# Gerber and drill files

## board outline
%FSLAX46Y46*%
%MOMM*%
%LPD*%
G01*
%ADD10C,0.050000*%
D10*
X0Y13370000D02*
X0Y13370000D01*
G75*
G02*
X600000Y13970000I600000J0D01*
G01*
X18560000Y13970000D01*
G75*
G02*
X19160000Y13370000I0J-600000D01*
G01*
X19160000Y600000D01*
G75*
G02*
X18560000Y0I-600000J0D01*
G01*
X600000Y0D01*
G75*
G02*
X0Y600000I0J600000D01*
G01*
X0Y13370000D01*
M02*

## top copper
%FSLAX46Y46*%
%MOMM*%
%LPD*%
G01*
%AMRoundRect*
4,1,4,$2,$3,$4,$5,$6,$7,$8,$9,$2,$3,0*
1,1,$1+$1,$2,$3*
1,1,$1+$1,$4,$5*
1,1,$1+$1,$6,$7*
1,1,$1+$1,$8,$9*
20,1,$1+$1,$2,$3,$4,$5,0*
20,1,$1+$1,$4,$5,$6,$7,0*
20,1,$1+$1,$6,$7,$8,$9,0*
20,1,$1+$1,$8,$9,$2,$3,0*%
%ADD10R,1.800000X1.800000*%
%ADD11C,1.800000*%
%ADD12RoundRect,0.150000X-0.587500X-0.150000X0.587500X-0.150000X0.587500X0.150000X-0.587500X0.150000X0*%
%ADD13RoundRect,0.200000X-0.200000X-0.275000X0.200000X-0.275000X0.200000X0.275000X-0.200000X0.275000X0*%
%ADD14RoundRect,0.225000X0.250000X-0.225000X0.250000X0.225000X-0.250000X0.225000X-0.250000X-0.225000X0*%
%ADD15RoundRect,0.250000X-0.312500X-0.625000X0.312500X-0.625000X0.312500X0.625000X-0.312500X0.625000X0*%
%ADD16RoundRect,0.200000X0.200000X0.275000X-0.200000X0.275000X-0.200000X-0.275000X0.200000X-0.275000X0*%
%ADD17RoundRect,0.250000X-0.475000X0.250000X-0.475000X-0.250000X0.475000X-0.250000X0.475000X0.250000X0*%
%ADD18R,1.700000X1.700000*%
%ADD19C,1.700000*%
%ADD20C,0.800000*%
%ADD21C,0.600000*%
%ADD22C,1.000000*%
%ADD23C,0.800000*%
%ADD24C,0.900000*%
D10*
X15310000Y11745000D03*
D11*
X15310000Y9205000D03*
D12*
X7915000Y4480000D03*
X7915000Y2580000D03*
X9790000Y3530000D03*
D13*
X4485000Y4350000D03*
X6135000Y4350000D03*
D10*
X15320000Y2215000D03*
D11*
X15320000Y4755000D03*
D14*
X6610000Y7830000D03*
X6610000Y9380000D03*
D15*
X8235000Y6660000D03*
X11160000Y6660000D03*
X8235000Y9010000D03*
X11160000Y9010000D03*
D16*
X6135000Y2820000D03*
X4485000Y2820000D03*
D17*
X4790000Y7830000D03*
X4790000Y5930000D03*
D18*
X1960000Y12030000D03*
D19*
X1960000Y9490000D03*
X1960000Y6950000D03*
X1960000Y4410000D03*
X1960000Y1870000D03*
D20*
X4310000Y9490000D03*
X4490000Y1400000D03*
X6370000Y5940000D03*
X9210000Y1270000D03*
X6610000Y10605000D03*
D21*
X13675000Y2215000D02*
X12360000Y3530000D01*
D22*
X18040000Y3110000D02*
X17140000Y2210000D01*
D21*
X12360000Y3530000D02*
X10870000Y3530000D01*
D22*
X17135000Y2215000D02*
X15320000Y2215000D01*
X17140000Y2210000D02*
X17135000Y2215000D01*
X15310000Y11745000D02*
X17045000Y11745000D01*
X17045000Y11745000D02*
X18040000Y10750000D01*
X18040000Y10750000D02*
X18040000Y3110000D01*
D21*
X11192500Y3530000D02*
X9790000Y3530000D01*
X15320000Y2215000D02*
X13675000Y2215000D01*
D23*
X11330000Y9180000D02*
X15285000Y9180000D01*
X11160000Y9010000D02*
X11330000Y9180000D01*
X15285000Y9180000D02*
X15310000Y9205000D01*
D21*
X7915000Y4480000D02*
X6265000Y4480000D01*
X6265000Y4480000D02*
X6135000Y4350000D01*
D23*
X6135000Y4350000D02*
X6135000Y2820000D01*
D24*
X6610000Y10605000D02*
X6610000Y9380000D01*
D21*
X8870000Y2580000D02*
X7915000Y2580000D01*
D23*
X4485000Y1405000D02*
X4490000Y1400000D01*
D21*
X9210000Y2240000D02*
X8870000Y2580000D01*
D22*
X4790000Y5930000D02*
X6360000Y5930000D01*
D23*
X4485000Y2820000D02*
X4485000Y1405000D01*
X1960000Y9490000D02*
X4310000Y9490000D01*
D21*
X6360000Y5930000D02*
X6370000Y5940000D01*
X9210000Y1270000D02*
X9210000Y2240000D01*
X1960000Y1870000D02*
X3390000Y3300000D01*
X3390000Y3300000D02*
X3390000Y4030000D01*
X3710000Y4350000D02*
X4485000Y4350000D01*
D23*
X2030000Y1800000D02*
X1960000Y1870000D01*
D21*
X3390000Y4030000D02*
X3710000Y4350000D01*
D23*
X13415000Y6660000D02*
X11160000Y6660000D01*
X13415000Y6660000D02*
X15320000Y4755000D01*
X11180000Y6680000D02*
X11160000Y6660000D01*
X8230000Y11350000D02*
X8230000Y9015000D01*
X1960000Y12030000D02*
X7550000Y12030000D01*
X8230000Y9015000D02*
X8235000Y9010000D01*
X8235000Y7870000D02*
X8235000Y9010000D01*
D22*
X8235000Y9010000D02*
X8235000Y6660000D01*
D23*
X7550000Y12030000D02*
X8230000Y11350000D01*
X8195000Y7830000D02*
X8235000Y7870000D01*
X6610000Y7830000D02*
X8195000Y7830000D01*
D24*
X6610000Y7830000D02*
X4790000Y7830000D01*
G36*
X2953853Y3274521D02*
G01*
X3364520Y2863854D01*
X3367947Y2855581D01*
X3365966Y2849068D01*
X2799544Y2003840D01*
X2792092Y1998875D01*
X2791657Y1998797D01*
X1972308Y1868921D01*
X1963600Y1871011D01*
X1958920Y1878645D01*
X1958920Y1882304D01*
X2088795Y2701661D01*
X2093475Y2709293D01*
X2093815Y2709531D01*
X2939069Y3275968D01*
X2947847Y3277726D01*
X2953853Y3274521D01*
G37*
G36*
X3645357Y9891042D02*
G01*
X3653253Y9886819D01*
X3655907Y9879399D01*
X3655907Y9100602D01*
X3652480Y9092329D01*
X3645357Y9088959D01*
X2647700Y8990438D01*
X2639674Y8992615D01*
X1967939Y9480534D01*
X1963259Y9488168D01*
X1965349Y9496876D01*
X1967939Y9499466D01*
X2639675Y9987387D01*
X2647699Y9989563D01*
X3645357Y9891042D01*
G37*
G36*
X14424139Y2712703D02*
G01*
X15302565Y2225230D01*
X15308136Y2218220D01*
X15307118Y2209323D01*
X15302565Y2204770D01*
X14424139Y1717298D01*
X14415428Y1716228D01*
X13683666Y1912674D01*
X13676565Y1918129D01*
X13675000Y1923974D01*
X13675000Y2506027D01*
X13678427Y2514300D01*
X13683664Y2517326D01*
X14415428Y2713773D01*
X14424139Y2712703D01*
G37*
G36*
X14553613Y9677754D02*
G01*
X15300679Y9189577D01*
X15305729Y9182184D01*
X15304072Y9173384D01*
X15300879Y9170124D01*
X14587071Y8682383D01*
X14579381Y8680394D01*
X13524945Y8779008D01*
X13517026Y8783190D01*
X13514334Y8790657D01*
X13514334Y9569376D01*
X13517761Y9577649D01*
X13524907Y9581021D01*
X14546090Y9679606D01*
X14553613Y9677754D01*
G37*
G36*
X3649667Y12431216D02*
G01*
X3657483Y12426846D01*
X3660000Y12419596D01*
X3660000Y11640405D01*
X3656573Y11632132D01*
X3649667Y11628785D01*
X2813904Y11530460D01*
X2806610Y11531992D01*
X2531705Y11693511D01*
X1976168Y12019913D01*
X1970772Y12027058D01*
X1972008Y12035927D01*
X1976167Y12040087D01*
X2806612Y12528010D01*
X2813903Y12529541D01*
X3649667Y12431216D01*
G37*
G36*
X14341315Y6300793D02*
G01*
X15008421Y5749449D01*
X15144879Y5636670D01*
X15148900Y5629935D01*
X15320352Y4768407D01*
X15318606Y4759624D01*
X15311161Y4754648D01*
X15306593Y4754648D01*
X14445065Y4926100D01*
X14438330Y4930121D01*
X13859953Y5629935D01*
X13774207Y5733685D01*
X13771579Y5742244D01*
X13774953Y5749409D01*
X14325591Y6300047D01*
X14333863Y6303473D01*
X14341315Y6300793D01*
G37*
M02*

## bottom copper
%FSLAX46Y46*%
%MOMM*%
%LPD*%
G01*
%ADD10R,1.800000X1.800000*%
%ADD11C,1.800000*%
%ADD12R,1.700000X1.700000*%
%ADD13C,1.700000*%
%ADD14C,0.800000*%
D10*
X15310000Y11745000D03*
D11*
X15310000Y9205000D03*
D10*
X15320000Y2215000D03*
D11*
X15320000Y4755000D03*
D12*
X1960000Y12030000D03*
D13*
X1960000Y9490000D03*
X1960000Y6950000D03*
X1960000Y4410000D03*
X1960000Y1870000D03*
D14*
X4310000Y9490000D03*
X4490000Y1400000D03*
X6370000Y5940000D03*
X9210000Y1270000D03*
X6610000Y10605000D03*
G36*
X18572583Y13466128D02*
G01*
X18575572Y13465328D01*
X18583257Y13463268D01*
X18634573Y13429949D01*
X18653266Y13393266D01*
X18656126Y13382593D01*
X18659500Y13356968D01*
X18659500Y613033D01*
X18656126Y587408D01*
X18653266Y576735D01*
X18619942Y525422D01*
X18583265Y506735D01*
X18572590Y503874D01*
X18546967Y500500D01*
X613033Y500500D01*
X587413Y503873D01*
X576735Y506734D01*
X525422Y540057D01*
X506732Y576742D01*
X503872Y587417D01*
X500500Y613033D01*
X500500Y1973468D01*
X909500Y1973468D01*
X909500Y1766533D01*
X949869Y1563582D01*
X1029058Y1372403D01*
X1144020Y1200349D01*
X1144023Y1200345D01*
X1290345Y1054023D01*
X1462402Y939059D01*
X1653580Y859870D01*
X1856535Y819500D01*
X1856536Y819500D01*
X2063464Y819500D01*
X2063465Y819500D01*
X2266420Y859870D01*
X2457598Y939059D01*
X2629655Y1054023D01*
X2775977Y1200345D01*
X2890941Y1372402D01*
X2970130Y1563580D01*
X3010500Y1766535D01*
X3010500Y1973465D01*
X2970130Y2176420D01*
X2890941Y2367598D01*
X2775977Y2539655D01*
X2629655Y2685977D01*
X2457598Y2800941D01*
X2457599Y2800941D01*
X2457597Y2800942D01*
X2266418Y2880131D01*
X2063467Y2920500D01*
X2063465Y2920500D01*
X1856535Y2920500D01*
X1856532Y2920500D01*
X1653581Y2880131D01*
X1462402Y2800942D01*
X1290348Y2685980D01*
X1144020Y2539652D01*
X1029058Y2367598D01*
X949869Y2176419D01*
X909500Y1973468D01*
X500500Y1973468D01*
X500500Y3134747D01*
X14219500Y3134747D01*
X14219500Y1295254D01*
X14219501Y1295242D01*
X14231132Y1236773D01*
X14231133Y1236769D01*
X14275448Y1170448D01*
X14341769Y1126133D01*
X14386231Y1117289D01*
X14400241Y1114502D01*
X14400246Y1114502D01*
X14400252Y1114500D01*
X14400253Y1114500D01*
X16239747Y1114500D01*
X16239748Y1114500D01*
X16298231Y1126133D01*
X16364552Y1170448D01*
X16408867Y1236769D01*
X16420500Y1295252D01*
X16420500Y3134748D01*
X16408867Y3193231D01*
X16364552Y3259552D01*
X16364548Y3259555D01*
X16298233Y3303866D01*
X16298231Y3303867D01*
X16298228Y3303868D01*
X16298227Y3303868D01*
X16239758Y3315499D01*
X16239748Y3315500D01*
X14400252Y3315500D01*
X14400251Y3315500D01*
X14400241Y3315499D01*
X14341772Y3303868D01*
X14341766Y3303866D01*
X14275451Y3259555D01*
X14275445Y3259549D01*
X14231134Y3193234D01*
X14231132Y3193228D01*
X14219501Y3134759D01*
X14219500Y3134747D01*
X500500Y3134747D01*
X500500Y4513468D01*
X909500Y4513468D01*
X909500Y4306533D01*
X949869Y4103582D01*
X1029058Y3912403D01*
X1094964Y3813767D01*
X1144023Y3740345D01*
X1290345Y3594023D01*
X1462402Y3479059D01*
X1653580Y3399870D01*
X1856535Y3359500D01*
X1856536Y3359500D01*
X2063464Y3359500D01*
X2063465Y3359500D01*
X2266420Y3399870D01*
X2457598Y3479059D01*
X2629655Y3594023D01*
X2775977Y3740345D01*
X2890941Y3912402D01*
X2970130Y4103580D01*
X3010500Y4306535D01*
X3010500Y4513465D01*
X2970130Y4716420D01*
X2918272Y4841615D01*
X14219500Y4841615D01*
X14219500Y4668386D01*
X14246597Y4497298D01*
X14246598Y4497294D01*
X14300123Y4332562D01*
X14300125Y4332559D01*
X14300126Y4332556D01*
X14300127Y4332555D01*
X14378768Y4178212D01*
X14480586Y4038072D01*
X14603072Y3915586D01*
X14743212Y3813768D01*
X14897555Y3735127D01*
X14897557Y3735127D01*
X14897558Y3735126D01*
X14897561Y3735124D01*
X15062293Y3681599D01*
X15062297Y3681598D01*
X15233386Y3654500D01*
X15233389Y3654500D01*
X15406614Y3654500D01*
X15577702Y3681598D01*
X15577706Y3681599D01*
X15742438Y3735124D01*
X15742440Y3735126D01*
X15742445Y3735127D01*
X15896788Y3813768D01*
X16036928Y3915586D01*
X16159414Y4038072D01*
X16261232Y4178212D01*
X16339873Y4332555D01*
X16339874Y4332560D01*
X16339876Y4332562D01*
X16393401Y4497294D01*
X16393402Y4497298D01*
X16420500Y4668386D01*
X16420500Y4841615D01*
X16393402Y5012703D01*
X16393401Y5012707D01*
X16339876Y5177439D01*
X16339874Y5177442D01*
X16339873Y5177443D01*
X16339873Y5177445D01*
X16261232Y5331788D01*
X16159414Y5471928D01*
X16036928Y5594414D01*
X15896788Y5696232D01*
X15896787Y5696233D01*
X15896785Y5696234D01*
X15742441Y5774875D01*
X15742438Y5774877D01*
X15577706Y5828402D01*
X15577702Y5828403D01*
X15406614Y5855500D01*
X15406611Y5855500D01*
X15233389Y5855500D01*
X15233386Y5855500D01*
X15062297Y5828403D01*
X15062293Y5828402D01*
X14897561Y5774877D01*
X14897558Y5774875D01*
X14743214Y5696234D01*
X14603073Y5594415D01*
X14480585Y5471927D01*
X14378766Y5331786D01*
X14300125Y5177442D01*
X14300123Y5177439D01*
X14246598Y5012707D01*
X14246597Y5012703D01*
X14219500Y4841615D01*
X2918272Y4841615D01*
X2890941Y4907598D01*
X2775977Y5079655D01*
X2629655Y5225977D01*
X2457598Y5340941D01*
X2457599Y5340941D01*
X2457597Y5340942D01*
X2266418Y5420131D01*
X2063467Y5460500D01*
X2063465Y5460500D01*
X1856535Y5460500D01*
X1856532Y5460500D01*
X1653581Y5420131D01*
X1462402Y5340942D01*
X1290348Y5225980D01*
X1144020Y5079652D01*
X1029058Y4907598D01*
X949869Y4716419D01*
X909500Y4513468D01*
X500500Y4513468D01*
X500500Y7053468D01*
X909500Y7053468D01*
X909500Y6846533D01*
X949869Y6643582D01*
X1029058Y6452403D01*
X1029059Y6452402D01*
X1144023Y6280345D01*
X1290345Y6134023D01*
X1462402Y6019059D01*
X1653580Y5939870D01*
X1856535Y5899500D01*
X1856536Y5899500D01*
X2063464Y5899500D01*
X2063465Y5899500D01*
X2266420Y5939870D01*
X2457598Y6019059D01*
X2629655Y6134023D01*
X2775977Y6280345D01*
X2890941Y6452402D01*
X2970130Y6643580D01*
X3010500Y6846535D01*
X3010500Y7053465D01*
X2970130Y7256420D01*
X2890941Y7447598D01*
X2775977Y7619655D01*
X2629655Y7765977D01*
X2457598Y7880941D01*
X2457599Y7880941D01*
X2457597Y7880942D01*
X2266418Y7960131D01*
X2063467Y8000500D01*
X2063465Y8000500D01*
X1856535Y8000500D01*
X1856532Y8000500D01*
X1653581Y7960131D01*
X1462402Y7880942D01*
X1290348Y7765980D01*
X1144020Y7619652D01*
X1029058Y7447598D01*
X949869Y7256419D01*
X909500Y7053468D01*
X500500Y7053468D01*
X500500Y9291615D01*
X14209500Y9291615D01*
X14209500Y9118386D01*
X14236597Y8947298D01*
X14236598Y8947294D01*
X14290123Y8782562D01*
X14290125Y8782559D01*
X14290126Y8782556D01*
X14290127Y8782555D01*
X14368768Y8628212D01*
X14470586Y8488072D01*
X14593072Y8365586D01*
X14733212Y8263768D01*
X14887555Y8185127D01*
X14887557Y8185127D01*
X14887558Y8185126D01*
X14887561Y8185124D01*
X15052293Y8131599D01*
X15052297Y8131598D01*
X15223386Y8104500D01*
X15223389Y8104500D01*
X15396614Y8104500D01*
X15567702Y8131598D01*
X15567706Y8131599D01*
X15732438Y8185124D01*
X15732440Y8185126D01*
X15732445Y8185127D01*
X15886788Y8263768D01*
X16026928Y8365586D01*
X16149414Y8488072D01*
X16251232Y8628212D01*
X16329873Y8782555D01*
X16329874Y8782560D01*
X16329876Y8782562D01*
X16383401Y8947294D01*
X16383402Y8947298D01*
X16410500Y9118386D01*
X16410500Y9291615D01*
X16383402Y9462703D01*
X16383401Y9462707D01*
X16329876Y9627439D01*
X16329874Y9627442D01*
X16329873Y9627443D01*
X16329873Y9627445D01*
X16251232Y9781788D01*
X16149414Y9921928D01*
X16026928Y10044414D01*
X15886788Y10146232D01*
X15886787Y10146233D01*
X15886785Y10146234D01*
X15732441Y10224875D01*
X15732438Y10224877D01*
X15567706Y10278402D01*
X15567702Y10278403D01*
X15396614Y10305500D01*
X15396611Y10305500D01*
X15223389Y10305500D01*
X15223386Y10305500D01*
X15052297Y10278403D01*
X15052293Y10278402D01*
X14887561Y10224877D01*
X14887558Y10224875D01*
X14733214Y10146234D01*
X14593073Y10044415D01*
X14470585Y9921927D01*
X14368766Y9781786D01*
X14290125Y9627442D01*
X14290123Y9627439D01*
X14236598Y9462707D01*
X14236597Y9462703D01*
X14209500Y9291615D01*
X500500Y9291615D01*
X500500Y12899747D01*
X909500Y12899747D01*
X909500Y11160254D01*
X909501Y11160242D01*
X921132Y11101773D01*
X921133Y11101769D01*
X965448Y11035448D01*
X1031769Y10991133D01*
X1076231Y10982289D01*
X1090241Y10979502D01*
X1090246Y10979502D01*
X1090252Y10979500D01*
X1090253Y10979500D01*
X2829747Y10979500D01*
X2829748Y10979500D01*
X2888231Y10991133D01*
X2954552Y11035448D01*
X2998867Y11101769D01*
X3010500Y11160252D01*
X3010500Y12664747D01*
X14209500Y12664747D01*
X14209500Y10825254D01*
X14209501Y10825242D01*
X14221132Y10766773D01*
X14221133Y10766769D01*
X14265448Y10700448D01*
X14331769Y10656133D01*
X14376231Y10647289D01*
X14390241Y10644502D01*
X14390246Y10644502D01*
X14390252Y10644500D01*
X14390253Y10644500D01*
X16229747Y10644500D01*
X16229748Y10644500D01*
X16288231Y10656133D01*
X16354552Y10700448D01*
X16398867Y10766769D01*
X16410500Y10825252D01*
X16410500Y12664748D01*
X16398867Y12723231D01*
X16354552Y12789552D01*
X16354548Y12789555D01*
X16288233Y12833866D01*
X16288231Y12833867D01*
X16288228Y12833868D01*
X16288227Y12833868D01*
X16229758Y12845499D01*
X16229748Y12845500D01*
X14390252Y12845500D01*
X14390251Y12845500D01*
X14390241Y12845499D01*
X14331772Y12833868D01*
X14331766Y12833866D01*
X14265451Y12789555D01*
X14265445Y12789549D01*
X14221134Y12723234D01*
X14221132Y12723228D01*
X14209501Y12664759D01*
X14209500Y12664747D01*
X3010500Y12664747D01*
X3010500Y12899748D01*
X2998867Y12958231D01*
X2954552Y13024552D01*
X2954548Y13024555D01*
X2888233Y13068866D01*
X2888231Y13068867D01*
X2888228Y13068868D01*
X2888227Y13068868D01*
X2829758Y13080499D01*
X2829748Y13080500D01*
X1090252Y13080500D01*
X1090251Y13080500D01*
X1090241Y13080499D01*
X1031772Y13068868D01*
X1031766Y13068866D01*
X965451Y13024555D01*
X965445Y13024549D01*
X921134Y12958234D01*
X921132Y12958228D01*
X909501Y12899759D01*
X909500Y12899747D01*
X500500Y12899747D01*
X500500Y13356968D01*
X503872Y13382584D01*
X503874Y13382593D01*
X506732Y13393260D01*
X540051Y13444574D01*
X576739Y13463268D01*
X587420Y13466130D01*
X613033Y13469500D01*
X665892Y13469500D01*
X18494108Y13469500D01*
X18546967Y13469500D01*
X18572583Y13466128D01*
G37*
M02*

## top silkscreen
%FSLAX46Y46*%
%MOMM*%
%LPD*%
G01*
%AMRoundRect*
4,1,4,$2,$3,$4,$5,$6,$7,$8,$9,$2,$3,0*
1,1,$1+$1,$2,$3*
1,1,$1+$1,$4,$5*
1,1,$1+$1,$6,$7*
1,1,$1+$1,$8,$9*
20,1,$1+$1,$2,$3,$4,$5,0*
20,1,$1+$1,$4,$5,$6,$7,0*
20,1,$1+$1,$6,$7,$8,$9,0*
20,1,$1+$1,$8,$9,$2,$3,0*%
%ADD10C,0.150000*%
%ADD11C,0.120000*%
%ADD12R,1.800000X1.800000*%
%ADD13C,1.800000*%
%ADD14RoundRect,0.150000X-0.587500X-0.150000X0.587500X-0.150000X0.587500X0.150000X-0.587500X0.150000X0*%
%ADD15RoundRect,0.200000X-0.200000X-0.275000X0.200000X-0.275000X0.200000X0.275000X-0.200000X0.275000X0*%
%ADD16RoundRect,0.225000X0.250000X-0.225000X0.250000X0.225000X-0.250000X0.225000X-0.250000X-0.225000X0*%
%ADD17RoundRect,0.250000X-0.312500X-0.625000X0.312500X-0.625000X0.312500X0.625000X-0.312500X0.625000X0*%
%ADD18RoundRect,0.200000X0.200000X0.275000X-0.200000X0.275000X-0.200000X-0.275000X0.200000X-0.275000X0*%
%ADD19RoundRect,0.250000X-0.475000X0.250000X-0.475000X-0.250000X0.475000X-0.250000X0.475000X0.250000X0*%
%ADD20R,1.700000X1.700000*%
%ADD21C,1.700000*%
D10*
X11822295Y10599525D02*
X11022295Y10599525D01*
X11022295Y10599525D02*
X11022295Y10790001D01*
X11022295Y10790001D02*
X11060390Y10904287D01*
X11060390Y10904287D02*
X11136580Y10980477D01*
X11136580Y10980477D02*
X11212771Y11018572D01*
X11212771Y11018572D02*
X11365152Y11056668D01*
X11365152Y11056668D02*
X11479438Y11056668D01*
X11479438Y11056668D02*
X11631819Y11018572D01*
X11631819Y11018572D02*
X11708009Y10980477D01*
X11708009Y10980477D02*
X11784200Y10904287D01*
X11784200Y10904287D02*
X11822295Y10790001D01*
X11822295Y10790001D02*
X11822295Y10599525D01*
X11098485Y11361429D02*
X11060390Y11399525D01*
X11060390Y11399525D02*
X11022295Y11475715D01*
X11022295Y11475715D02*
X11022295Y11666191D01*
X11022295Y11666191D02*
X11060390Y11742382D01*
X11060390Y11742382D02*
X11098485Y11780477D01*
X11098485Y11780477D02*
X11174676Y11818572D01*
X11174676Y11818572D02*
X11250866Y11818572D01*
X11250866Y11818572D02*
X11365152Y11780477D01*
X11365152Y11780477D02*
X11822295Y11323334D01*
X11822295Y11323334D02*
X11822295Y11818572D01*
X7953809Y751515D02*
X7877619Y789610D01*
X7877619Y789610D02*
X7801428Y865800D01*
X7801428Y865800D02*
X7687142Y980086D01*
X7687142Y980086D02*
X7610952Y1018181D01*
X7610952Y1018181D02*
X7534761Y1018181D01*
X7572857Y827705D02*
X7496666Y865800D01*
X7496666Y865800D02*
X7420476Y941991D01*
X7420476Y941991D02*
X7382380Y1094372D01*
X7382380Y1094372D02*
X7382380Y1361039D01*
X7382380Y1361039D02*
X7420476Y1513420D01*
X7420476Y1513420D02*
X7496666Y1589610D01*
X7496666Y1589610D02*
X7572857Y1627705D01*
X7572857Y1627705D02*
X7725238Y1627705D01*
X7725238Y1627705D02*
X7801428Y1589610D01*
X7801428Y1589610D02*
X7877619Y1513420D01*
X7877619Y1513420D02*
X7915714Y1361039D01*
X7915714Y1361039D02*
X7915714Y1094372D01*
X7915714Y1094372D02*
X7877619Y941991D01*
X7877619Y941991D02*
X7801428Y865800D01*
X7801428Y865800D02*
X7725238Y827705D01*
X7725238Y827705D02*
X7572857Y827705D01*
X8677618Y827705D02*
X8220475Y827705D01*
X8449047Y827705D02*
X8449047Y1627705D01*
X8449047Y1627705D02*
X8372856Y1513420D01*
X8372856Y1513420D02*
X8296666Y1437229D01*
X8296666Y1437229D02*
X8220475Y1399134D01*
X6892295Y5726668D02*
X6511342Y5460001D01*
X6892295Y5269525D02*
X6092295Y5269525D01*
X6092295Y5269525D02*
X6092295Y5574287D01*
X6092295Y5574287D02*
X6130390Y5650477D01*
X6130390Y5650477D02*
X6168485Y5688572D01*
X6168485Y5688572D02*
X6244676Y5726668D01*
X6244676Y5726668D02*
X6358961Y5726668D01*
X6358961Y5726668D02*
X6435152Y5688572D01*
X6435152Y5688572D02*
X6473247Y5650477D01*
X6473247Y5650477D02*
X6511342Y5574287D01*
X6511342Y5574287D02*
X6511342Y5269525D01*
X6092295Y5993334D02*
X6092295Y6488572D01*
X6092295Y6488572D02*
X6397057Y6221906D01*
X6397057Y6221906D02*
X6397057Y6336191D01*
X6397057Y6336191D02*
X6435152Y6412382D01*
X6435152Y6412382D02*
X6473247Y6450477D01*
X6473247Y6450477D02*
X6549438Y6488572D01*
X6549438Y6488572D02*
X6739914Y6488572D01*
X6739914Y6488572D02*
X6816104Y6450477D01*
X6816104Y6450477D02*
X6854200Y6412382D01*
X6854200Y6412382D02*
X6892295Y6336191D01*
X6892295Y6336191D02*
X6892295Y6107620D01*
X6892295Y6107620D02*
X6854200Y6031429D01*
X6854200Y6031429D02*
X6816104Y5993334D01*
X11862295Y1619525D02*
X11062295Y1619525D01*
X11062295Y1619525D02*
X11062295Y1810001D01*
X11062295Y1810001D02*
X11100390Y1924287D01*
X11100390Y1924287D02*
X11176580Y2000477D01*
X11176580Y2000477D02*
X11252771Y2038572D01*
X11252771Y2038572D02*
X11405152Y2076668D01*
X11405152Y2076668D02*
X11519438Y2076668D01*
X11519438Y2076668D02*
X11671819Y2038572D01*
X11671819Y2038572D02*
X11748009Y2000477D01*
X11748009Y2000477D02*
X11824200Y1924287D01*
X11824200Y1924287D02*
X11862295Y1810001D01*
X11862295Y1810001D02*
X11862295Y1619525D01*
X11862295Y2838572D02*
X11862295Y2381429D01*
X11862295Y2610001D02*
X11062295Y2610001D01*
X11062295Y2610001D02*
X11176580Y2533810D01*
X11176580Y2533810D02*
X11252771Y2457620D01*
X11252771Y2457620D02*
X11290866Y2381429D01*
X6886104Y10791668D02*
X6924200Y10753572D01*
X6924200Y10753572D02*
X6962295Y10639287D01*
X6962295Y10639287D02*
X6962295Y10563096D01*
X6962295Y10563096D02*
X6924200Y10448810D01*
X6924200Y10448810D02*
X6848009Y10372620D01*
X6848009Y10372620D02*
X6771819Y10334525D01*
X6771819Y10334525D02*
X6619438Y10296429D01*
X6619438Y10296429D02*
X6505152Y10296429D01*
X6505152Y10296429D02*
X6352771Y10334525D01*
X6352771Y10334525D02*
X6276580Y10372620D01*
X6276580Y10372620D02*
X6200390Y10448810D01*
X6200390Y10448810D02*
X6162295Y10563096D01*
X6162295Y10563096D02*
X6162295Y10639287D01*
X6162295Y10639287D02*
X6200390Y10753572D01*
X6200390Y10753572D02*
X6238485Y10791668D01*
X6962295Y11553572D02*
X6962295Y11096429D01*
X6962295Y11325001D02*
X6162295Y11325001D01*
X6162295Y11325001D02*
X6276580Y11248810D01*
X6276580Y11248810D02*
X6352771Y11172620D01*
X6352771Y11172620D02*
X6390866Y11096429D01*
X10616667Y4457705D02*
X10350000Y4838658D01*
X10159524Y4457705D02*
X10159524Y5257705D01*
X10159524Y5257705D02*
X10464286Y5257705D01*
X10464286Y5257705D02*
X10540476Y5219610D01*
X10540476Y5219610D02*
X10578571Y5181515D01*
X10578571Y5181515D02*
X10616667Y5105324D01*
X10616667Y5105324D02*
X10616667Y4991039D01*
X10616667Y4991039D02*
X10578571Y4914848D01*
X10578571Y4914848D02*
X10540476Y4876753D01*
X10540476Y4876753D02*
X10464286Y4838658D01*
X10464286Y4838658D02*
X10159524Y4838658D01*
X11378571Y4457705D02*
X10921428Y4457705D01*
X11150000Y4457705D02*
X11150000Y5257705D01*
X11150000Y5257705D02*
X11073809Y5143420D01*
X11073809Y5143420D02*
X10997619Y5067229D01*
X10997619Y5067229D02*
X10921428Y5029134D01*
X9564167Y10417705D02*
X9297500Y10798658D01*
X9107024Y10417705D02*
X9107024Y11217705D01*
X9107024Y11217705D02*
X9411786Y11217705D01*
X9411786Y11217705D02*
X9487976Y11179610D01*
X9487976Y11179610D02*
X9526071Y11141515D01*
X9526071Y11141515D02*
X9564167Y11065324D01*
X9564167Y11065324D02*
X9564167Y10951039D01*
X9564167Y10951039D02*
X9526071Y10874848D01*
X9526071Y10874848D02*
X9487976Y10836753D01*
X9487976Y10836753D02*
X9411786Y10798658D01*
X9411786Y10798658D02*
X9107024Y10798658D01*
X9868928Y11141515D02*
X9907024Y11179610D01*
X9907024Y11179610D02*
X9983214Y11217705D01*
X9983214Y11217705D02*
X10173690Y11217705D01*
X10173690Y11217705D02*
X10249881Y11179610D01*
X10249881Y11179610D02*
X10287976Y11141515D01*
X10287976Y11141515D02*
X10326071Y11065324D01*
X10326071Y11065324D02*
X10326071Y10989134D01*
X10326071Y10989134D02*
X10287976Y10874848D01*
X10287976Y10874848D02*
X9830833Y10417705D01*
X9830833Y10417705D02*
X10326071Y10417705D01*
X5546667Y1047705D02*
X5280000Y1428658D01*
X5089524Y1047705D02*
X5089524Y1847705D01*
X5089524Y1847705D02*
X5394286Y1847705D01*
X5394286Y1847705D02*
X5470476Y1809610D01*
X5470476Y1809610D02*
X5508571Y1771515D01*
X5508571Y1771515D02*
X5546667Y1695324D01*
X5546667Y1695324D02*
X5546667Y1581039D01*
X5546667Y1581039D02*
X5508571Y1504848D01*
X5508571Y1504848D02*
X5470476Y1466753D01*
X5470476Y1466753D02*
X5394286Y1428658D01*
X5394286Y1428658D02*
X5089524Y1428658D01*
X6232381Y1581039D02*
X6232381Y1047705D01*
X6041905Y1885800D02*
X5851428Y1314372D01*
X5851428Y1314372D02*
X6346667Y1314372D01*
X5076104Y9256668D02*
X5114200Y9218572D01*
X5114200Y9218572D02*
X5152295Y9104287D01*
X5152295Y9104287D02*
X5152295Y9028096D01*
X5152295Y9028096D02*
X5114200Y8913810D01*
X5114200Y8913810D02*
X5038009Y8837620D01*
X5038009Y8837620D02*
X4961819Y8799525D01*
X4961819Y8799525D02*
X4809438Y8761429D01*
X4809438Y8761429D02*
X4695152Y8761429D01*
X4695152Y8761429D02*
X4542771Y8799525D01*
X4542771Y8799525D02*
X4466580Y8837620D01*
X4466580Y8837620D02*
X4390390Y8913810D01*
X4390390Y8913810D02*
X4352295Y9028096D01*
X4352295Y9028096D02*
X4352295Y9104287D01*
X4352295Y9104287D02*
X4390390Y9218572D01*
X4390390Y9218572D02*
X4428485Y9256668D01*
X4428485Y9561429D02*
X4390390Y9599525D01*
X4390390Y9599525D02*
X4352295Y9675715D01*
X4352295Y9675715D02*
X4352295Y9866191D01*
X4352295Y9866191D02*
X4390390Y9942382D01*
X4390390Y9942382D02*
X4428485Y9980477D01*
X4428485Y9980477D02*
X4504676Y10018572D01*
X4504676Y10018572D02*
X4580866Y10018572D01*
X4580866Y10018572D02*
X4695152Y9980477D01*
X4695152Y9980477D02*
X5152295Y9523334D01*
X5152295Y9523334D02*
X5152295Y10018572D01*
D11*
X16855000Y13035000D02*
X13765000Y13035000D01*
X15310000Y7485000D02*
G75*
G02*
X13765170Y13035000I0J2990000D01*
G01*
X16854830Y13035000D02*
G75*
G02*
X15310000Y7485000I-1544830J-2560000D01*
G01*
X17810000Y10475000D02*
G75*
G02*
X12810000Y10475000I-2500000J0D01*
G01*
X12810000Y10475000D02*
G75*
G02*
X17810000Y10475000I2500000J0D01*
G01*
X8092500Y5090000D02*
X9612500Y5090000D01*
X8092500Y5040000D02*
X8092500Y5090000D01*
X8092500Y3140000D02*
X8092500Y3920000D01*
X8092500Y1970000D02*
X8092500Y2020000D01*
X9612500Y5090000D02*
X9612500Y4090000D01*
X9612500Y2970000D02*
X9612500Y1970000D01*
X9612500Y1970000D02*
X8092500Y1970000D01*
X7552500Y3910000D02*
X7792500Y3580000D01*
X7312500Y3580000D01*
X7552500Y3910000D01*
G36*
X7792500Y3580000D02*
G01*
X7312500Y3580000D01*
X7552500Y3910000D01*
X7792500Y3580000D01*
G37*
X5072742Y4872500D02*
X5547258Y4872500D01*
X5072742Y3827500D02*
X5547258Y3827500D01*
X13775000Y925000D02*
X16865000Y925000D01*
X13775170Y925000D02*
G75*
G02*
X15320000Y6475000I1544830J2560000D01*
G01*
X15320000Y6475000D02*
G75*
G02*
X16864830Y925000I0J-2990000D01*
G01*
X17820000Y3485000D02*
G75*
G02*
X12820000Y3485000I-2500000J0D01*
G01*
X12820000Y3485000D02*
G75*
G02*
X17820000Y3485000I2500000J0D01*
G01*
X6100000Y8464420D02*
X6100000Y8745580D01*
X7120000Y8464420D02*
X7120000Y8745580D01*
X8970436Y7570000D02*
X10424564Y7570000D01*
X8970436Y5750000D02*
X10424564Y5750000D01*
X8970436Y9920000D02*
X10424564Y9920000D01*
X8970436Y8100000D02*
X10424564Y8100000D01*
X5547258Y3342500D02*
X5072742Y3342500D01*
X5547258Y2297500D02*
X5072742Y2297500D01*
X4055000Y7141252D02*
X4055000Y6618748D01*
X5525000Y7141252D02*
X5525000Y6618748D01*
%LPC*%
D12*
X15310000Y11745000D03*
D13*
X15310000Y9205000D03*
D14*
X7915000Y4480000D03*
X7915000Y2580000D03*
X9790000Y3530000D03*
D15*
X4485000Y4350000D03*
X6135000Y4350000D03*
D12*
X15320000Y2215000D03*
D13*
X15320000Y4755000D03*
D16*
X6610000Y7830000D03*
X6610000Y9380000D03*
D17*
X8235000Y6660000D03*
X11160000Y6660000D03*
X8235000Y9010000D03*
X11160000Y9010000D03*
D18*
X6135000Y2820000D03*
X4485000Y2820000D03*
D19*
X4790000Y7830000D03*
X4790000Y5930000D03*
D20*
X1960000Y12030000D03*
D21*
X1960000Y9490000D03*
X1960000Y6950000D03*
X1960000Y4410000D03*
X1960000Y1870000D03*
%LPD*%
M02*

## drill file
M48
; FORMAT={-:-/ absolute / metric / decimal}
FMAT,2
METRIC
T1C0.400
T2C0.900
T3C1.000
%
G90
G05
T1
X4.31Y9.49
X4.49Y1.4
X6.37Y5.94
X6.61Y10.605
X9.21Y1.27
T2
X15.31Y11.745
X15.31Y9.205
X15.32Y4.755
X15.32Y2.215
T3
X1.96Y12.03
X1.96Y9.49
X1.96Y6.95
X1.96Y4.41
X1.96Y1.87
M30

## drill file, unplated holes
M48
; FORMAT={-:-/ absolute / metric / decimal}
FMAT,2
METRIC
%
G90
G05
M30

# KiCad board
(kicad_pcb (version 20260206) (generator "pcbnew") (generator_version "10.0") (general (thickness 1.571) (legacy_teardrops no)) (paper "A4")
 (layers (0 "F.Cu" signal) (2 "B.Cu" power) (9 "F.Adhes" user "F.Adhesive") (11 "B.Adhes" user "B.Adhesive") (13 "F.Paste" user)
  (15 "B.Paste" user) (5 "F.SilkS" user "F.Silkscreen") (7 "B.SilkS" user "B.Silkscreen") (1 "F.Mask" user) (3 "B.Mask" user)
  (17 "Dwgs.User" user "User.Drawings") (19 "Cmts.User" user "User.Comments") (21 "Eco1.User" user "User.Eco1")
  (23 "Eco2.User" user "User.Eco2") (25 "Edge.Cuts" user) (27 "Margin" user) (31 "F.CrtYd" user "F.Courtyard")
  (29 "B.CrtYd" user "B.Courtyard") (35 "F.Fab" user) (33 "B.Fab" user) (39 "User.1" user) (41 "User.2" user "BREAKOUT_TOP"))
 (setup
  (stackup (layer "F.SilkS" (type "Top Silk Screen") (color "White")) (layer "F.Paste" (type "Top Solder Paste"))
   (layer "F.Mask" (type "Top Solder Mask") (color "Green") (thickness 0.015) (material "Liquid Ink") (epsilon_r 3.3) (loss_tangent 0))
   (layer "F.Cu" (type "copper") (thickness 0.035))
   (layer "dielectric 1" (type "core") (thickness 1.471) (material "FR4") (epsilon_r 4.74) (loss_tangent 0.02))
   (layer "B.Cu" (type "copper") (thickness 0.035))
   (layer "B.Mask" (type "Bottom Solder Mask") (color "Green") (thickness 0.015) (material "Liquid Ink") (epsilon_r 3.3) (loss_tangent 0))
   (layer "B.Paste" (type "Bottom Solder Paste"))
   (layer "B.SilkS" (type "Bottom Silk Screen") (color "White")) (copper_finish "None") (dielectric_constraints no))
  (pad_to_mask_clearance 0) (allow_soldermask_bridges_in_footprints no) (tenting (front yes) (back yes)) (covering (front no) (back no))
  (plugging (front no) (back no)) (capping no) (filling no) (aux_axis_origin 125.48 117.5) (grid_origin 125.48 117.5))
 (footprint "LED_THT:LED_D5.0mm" (layer "F.Cu") (at 140.79 105.755 -90)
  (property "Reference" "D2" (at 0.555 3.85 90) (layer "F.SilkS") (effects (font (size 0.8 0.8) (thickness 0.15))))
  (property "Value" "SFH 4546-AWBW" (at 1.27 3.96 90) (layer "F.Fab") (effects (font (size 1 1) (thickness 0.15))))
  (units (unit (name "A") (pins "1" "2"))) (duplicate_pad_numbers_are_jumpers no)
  (fp_line (start -1.29 -1.545) (end -1.29 1.545) (stroke (width 0.12) (type solid)) (layer "F.SilkS"))
  (fp_arc (start 4.26 0) (mid 2.071779 2.880495) (end -1.29 1.54483) (stroke (width 0.12) (type solid)) (layer "F.SilkS"))
  (fp_arc (start -1.29 -1.54483) (mid 2.071779 -2.880495) (end 4.26 0) (stroke (width 0.12) (type solid)) (layer "F.SilkS"))
  (fp_circle (center 1.27 0) (end 3.77 0) (stroke (width 0.12) (type solid)) (fill no) (layer "F.SilkS"))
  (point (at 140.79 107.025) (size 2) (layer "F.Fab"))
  (pad "1" thru_hole rect (at 0 0 270) (size 1.8 1.8) (drill 0.9) (layers "*.Cu" "*.Mask") (remove_unused_layers no) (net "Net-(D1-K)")
   (teardrops (best_length_ratio 0.5) (max_length 1) (best_width_ratio 1) (max_width 1) (curved_edges no) (filter_ratio 0.9) (enabled yes)
    (allow_two_segments no) (prefer_zone_connections yes)))
  (pad "2" thru_hole circle (at 2.54 0 270) (size 1.8 1.8) (drill 0.9) (layers "*.Cu" "*.Mask") (remove_unused_layers no) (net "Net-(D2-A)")
   (teardrops (best_length_ratio 0.5) (max_length 1) (best_width_ratio 1) (max_width 1) (curved_edges no) (filter_ratio 0.9) (enabled yes)
    (allow_two_segments no) (prefer_zone_connections yes))))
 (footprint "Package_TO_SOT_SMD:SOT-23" (layer "F.Cu") (at 134.3325 113.97)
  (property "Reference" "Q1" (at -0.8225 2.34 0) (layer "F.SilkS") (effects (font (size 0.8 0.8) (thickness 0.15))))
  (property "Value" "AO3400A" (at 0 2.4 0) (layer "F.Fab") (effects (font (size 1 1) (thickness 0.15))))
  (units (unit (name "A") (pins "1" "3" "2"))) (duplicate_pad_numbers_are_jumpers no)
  (fp_line (start -0.76 -1.56) (end 0.76 -1.56) (stroke (width 0.12) (type solid)) (layer "F.SilkS"))
  (fp_line (start -0.76 -1.51) (end -0.76 -1.56) (stroke (width 0.12) (type solid)) (layer "F.SilkS"))
  (fp_line (start -0.76 0.39) (end -0.76 -0.39) (stroke (width 0.12) (type solid)) (layer "F.SilkS"))
  (fp_line (start -0.76 1.56) (end -0.76 1.51) (stroke (width 0.12) (type solid)) (layer "F.SilkS"))
  (fp_line (start 0.76 -1.56) (end 0.76 -0.56) (stroke (width 0.12) (type solid)) (layer "F.SilkS"))
  (fp_line (start 0.76 0.56) (end 0.76 1.56) (stroke (width 0.12) (type solid)) (layer "F.SilkS"))
  (fp_line (start 0.76 1.56) (end -0.76 1.56) (stroke (width 0.12) (type solid)) (layer "F.SilkS"))
  (fp_poly (pts (xy -1.3 -0.38) (xy -1.06 -0.05) (xy -1.54 -0.05)) (stroke (width 0.12) (type solid)) (fill yes) (layer "F.SilkS"))
  (pad "1" smd roundrect (at -0.9375 -0.95) (size 1.475 0.6) (layers "F.Cu" "F.Mask" "F.Paste") (roundrect_rratio 0.25) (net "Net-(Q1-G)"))
  (pad "2" smd roundrect (at -0.9375 0.95) (size 1.475 0.6) (layers "F.Cu" "F.Mask" "F.Paste") (roundrect_rratio 0.25) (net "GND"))
  (pad "3" smd roundrect (at 0.9375 0) (size 1.475 0.6) (layers "F.Cu" "F.Mask" "F.Paste") (roundrect_rratio 0.25) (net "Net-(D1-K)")))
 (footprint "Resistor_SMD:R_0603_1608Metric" (layer "F.Cu") (at 130.79 113.15)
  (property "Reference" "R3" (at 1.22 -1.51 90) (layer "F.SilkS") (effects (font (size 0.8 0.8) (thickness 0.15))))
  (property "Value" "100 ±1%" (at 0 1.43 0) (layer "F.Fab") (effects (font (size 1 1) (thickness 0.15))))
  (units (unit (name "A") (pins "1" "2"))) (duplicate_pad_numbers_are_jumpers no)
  (fp_line (start -0.237258 -0.5225) (end 0.237258 -0.5225) (stroke (width 0.12) (type solid)) (layer "F.SilkS"))
  (fp_line (start -0.237258 0.5225) (end 0.237258 0.5225) (stroke (width 0.12) (type solid)) (layer "F.SilkS"))
  (pad "1" smd roundrect (at -0.825 0) (size 0.8 0.95) (layers "F.Cu" "F.Mask" "F.Paste") (roundrect_rratio 0.25) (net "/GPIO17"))
  (pad "2" smd roundrect (at 0.825 0) (size 0.8 0.95) (layers "F.Cu" "F.Mask" "F.Paste") (roundrect_rratio 0.25) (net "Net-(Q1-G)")))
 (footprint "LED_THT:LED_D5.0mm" (layer "F.Cu") (at 140.8 115.285 90)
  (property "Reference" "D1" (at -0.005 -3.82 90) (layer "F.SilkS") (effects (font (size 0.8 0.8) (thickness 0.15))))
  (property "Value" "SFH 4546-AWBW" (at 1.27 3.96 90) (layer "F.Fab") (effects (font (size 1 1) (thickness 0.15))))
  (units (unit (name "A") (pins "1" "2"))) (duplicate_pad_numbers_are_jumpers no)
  (fp_line (start -1.29 -1.545) (end -1.29 1.545) (stroke (width 0.12) (type solid)) (layer "F.SilkS"))
  (fp_arc (start -1.29 -1.54483) (mid 2.071779 -2.880495) (end 4.26 0) (stroke (width 0.12) (type solid)) (layer "F.SilkS"))
  (fp_arc (start 4.26 0) (mid 2.071779 2.880495) (end -1.29 1.54483) (stroke (width 0.12) (type solid)) (layer "F.SilkS"))
  (fp_circle (center 1.27 0) (end 3.77 0) (stroke (width 0.12) (type solid)) (fill no) (layer "F.SilkS"))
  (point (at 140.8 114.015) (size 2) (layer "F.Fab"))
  (pad "1" thru_hole rect (at 0 0 90) (size 1.8 1.8) (drill 0.9) (layers "*.Cu" "*.Mask") (remove_unused_layers no) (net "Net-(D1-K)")
   (teardrops (best_length_ratio 0.5) (max_length 1) (best_width_ratio 1) (max_width 1) (curved_edges no) (filter_ratio 0.9) (enabled yes)
    (allow_two_segments no) (prefer_zone_connections yes)))
  (pad "2" thru_hole circle (at 2.54 0 90) (size 1.8 1.8) (drill 0.9) (layers "*.Cu" "*.Mask") (remove_unused_layers no) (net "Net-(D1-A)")
   (teardrops (best_length_ratio 0.5) (max_length 1) (best_width_ratio 1) (max_width 1) (curved_edges no) (filter_ratio 0.9) (enabled yes)
    (allow_two_segments no) (prefer_zone_connections yes))))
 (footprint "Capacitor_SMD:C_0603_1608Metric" (layer "F.Cu") (at 132.09 108.895 90)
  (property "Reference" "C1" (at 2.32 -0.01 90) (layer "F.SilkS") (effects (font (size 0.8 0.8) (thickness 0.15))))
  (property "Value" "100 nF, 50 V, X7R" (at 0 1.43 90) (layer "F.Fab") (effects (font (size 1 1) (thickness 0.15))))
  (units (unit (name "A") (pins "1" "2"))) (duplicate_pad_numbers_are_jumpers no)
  (fp_line (start -0.14058 -0.51) (end 0.14058 -0.51) (stroke (width 0.12) (type solid)) (layer "F.SilkS"))
  (fp_line (start -0.14058 0.51) (end 0.14058 0.51) (stroke (width 0.12) (type solid)) (layer "F.SilkS"))
  (pad "1" smd roundrect (at -0.775 0 90) (size 0.9 0.95) (layers "F.Cu" "F.Mask" "F.Paste") (roundrect_rratio 0.25) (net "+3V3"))
  (pad "2" smd roundrect (at 0.775 0 90) (size 0.9 0.95) (layers "F.Cu" "F.Mask" "F.Paste") (roundrect_rratio 0.25) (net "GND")))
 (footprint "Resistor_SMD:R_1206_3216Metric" (layer "F.Cu") (at 135.1775 110.84)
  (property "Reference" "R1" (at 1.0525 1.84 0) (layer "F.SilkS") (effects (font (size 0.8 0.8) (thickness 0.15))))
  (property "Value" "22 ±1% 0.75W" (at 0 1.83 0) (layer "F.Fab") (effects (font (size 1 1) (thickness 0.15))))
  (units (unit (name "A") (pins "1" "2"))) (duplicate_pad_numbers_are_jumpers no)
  (fp_line (start -0.727064 -0.91) (end 0.727064 -0.91) (stroke (width 0.12) (type solid)) (layer "F.SilkS"))
  (fp_line (start -0.727064 0.91) (end 0.727064 0.91) (stroke (width 0.12) (type solid)) (layer "F.SilkS"))
  (pad "1" smd roundrect (at -1.4625 0) (size 1.125 1.75) (layers "F.Cu" "F.Mask" "F.Paste") (roundrect_rratio 0.222222) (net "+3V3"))
  (pad "2" smd roundrect (at 1.4625 0) (size 1.125 1.75) (layers "F.Cu" "F.Mask" "F.Paste") (roundrect_rratio 0.222222) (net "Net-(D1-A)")))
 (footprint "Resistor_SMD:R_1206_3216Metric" (layer "F.Cu") (at 135.1775 108.49)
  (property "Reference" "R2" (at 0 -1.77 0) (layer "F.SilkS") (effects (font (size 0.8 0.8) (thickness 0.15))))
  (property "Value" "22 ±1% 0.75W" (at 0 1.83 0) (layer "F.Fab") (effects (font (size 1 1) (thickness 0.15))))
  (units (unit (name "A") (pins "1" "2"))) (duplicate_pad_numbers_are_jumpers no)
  (fp_line (start -0.727064 -0.91) (end 0.727064 -0.91) (stroke (width 0.12) (type solid)) (layer "F.SilkS"))
  (fp_line (start -0.727064 0.91) (end 0.727064 0.91) (stroke (width 0.12) (type solid)) (layer "F.SilkS"))
  (pad "1" smd roundrect (at -1.4625 0) (size 1.125 1.75) (layers "F.Cu" "F.Mask" "F.Paste") (roundrect_rratio 0.222222) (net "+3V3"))
  (pad "2" smd roundrect (at 1.4625 0) (size 1.125 1.75) (layers "F.Cu" "F.Mask" "F.Paste") (roundrect_rratio 0.222222) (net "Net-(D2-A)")))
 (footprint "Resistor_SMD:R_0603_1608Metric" (layer "F.Cu") (at 130.79 114.68 180)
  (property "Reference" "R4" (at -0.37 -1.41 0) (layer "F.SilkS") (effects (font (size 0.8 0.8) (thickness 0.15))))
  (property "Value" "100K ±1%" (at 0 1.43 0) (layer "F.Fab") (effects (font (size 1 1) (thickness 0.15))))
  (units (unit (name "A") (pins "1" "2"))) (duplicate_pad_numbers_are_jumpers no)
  (fp_line (start -0.237258 0.5225) (end 0.237258 0.5225) (stroke (width 0.12) (type solid)) (layer "F.SilkS"))
  (fp_line (start -0.237258 -0.5225) (end 0.237258 -0.5225) (stroke (width 0.12) (type solid)) (layer "F.SilkS"))
  (pad "1" smd roundrect (at -0.825 0 180) (size 0.8 0.95) (layers "F.Cu" "F.Mask" "F.Paste") (roundrect_rratio 0.25) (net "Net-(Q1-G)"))
  (pad "2" smd roundrect (at 0.825 0 180) (size 0.8 0.95) (layers "F.Cu" "F.Mask" "F.Paste") (roundrect_rratio 0.25) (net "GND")))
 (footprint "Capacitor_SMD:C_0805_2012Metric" (layer "F.Cu") (at 130.27 110.62 -90)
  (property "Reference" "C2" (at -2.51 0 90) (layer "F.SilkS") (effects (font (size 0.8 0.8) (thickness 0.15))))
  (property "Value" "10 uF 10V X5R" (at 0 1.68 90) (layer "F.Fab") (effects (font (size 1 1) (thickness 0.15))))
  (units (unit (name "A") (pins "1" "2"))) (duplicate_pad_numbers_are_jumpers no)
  (fp_line (start -0.261252 0.735) (end 0.261252 0.735) (stroke (width 0.12) (type solid)) (layer "F.SilkS"))
  (fp_line (start -0.261252 -0.735) (end 0.261252 -0.735) (stroke (width 0.12) (type solid)) (layer "F.SilkS"))
  (pad "1" smd roundrect (at -0.95 0 270) (size 1 1.45) (layers "F.Cu" "F.Mask" "F.Paste") (roundrect_rratio 0.25) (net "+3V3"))
  (pad "2" smd roundrect (at 0.95 0 270) (size 1 1.45) (layers "F.Cu" "F.Mask" "F.Paste") (roundrect_rratio 0.25) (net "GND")))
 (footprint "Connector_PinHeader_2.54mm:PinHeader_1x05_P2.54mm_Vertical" (layer "B.Cu") (at 127.44 105.47 180)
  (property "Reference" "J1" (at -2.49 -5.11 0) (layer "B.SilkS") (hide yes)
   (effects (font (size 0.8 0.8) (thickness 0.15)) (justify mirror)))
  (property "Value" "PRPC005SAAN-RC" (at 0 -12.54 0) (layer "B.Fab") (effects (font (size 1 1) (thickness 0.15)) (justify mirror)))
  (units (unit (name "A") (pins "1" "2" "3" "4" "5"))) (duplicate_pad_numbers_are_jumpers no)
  (pad "1" thru_hole rect (at 0 0 180) (size 1.7 1.7) (drill 1) (layers "*.Cu" "*.Mask") (remove_unused_layers no) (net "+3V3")
   (teardrops (best_length_ratio 0.5) (max_length 1) (best_width_ratio 1) (max_width 1) (curved_edges no) (filter_ratio 0.9) (enabled yes)
    (allow_two_segments no) (prefer_zone_connections yes)))
  (pad "2" thru_hole circle (at 0 -2.54 180) (size 1.7 1.7) (drill 1) (layers "*.Cu" "*.Mask") (remove_unused_layers no) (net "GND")
   (teardrops (best_length_ratio 0.5) (max_length 1) (best_width_ratio 1) (max_width 1) (curved_edges no) (filter_ratio 0.9) (enabled yes)
    (allow_two_segments no) (prefer_zone_connections yes)))
  (pad "3" thru_hole circle (at 0 -5.08 180) (size 1.7 1.7) (drill 1) (layers "*.Cu" "*.Mask") (remove_unused_layers no)
   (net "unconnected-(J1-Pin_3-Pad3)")
   (teardrops (best_length_ratio 0.5) (max_length 1) (best_width_ratio 1) (max_width 1) (curved_edges no) (filter_ratio 0.9) (enabled yes)
    (allow_two_segments no) (prefer_zone_connections yes)))
  (pad "4" thru_hole circle (at 0 -7.62 180) (size 1.7 1.7) (drill 1) (layers "*.Cu" "*.Mask") (remove_unused_layers no)
   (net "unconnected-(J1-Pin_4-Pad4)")
   (teardrops (best_length_ratio 0.5) (max_length 1) (best_width_ratio 1) (max_width 1) (curved_edges no) (filter_ratio 0.9) (enabled yes)
    (allow_two_segments no) (prefer_zone_connections yes)))
  (pad "5" thru_hole circle (at 0 -10.16 180) (size 1.7 1.7) (drill 1) (layers "*.Cu" "*.Mask") (remove_unused_layers no) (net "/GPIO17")
   (teardrops (best_length_ratio 0.5) (max_length 1) (best_width_ratio 1) (max_width 1) (curved_edges no) (filter_ratio 0.9) (enabled yes)
    (allow_two_segments no) (prefer_zone_connections yes))))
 (gr_rect (start 125.48 103.53) (end 144.64 117.5) (radius 0.6) (stroke (width 0.05) (type solid)) (fill no) (layer "Edge.Cuts"))
 (segment (start 139.155 115.285) (end 137.84 113.97) (width 0.6) (layer "F.Cu") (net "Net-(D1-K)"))
 (segment (start 143.52 114.39) (end 142.62 115.29) (width 1) (layer "F.Cu") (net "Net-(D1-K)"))
 (segment (start 137.84 113.97) (end 136.35 113.97) (width 0.6) (layer "F.Cu") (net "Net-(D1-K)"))
 (segment (start 142.615 115.285) (end 140.8 115.285) (width 1) (layer "F.Cu") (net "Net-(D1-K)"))
 (segment (start 142.62 115.29) (end 142.615 115.285) (width 1) (layer "F.Cu") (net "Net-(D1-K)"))
 (segment (start 140.79 105.755) (end 142.525 105.755) (width 1) (layer "F.Cu") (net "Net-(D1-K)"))
 (segment (start 142.525 105.755) (end 143.52 106.75) (width 1) (layer "F.Cu") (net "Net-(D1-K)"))
 (segment (start 143.52 106.75) (end 143.52 114.39) (width 1) (layer "F.Cu") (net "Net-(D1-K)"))
 (segment (start 136.6725 113.97) (end 135.27 113.97) (width 0.6) (layer "F.Cu") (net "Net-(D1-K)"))
 (segment (start 140.8 115.285) (end 139.155 115.285) (width 0.6) (layer "F.Cu") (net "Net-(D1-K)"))
 (segment (start 136.81 108.32) (end 140.765 108.32) (width 0.8) (layer "F.Cu") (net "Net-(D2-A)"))
 (segment (start 136.64 108.49) (end 136.81 108.32) (width 0.8) (layer "F.Cu") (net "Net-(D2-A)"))
 (segment (start 140.765 108.32) (end 140.79 108.295) (width 0.8) (layer "F.Cu") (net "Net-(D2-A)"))
 (segment (start 133.395 113.02) (end 131.745 113.02) (width 0.6) (layer "F.Cu") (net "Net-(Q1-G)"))
 (segment (start 131.745 113.02) (end 131.615 113.15) (width 0.6) (layer "F.Cu") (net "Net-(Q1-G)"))
 (segment (start 131.615 113.15) (end 131.615 114.68) (width 0.8) (layer "F.Cu") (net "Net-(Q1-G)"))
 (segment (start 132.09 106.895) (end 132.09 108.12) (width 0.9) (layer "F.Cu") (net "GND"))
 (segment (start 134.35 114.92) (end 133.395 114.92) (width 0.6) (layer "F.Cu") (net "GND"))
 (segment (start 129.965 116.095) (end 129.97 116.1) (width 0.8) (layer "F.Cu") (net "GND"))
 (segment (start 134.69 115.26) (end 134.35 114.92) (width 0.6) (layer "F.Cu") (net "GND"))
 (segment (start 130.27 111.57) (end 131.84 111.57) (width 1) (layer "F.Cu") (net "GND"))
 (segment (start 129.965 114.68) (end 129.965 116.095) (width 0.8) (layer "F.Cu") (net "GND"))
 (segment (start 127.44 108.01) (end 129.79 108.01) (width 0.8) (layer "F.Cu") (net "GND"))
 (segment (start 131.84 111.57) (end 131.85 111.56) (width 0.6) (layer "F.Cu") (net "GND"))
 (segment (start 134.69 116.23) (end 134.69 115.26) (width 0.6) (layer "F.Cu") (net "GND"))
 (via (at 129.79 108.01) (size 0.8) (drill 0.4) (layers "F.Cu" "B.Cu") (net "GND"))
 (via (at 129.97 116.1) (size 0.8) (drill 0.4) (layers "F.Cu" "B.Cu") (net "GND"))
 (via (at 131.85 111.56) (size 0.8) (drill 0.4) (layers "F.Cu" "B.Cu") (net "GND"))
 (via (at 134.69 116.23) (size 0.8) (drill 0.4) (layers "F.Cu" "B.Cu") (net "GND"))
 (via (at 132.09 106.895) (size 0.8) (drill 0.4) (layers "F.Cu" "B.Cu") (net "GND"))
 (segment (start 127.44 115.63) (end 128.87 114.2) (width 0.6) (layer "F.Cu") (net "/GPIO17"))
 (segment (start 128.87 114.2) (end 128.87 113.47) (width 0.6) (layer "F.Cu") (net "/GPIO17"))
 (segment (start 129.19 113.15) (end 129.965 113.15) (width 0.6) (layer "F.Cu") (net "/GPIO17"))
 (segment (start 127.51 115.7) (end 127.44 115.63) (width 0.8) (layer "F.Cu") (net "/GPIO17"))
 (segment (start 128.87 113.47) (end 129.19 113.15) (width 0.6) (layer "F.Cu") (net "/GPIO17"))
 (segment (start 138.895 110.84) (end 136.64 110.84) (width 0.8) (layer "F.Cu") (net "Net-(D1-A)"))
 (segment (start 138.895 110.84) (end 140.8 112.745) (width 0.8) (layer "F.Cu") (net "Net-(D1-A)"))
 (segment (start 136.66 110.82) (end 136.64 110.84) (width 0.8) (layer "F.Cu") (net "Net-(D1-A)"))
 (segment (start 133.71 106.15) (end 133.71 108.485) (width 0.8) (layer "F.Cu") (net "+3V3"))
 (segment (start 127.44 105.47) (end 133.03 105.47) (width 0.8) (layer "F.Cu") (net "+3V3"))
 (segment (start 133.71 108.485) (end 133.715 108.49) (width 0.8) (layer "F.Cu") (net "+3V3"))
 (segment (start 133.715 109.63) (end 133.715 108.49) (width 0.8) (layer "F.Cu") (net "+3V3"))
 (segment (start 133.715 108.49) (end 133.715 110.84) (width 1) (layer "F.Cu") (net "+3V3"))
 (segment (start 133.03 105.47) (end 133.71 106.15) (width 0.8) (layer "F.Cu") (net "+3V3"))
 (segment (start 133.675 109.67) (end 133.715 109.63) (width 0.8) (layer "F.Cu") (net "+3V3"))
 (segment (start 132.09 109.67) (end 133.675 109.67) (width 0.8) (layer "F.Cu") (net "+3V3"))
 (segment (start 132.09 109.67) (end 130.27 109.67) (width 0.9) (layer "F.Cu") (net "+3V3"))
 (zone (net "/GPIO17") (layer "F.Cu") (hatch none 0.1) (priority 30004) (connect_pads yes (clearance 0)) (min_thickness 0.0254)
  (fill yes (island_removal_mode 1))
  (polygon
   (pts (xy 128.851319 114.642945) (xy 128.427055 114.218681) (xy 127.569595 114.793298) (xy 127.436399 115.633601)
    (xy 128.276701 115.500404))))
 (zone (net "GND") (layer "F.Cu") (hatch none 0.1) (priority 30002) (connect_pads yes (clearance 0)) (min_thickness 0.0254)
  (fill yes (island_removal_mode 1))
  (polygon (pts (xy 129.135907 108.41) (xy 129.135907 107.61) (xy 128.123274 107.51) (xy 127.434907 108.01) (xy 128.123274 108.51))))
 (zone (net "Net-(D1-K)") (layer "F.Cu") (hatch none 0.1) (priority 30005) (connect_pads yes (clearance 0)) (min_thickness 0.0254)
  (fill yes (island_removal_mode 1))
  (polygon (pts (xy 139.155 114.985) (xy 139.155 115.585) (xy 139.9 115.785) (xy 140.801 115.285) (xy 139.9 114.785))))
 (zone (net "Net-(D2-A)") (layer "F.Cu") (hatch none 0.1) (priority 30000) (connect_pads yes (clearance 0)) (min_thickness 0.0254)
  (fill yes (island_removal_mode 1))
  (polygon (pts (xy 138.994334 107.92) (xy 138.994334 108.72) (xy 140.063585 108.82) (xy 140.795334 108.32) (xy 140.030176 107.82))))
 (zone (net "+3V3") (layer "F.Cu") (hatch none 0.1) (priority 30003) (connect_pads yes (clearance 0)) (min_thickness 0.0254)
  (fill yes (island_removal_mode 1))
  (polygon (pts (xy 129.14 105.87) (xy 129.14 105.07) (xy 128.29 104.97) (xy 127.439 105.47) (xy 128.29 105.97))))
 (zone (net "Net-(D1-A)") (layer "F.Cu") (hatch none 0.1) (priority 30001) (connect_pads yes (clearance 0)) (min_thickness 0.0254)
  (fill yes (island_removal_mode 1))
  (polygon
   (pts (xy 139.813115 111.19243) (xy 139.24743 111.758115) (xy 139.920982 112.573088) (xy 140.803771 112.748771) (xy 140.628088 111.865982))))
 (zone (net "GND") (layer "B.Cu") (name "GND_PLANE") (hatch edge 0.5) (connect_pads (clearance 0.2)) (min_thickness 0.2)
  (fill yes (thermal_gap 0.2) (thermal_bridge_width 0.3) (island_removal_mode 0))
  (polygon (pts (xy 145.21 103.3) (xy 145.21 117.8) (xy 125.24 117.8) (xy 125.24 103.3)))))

